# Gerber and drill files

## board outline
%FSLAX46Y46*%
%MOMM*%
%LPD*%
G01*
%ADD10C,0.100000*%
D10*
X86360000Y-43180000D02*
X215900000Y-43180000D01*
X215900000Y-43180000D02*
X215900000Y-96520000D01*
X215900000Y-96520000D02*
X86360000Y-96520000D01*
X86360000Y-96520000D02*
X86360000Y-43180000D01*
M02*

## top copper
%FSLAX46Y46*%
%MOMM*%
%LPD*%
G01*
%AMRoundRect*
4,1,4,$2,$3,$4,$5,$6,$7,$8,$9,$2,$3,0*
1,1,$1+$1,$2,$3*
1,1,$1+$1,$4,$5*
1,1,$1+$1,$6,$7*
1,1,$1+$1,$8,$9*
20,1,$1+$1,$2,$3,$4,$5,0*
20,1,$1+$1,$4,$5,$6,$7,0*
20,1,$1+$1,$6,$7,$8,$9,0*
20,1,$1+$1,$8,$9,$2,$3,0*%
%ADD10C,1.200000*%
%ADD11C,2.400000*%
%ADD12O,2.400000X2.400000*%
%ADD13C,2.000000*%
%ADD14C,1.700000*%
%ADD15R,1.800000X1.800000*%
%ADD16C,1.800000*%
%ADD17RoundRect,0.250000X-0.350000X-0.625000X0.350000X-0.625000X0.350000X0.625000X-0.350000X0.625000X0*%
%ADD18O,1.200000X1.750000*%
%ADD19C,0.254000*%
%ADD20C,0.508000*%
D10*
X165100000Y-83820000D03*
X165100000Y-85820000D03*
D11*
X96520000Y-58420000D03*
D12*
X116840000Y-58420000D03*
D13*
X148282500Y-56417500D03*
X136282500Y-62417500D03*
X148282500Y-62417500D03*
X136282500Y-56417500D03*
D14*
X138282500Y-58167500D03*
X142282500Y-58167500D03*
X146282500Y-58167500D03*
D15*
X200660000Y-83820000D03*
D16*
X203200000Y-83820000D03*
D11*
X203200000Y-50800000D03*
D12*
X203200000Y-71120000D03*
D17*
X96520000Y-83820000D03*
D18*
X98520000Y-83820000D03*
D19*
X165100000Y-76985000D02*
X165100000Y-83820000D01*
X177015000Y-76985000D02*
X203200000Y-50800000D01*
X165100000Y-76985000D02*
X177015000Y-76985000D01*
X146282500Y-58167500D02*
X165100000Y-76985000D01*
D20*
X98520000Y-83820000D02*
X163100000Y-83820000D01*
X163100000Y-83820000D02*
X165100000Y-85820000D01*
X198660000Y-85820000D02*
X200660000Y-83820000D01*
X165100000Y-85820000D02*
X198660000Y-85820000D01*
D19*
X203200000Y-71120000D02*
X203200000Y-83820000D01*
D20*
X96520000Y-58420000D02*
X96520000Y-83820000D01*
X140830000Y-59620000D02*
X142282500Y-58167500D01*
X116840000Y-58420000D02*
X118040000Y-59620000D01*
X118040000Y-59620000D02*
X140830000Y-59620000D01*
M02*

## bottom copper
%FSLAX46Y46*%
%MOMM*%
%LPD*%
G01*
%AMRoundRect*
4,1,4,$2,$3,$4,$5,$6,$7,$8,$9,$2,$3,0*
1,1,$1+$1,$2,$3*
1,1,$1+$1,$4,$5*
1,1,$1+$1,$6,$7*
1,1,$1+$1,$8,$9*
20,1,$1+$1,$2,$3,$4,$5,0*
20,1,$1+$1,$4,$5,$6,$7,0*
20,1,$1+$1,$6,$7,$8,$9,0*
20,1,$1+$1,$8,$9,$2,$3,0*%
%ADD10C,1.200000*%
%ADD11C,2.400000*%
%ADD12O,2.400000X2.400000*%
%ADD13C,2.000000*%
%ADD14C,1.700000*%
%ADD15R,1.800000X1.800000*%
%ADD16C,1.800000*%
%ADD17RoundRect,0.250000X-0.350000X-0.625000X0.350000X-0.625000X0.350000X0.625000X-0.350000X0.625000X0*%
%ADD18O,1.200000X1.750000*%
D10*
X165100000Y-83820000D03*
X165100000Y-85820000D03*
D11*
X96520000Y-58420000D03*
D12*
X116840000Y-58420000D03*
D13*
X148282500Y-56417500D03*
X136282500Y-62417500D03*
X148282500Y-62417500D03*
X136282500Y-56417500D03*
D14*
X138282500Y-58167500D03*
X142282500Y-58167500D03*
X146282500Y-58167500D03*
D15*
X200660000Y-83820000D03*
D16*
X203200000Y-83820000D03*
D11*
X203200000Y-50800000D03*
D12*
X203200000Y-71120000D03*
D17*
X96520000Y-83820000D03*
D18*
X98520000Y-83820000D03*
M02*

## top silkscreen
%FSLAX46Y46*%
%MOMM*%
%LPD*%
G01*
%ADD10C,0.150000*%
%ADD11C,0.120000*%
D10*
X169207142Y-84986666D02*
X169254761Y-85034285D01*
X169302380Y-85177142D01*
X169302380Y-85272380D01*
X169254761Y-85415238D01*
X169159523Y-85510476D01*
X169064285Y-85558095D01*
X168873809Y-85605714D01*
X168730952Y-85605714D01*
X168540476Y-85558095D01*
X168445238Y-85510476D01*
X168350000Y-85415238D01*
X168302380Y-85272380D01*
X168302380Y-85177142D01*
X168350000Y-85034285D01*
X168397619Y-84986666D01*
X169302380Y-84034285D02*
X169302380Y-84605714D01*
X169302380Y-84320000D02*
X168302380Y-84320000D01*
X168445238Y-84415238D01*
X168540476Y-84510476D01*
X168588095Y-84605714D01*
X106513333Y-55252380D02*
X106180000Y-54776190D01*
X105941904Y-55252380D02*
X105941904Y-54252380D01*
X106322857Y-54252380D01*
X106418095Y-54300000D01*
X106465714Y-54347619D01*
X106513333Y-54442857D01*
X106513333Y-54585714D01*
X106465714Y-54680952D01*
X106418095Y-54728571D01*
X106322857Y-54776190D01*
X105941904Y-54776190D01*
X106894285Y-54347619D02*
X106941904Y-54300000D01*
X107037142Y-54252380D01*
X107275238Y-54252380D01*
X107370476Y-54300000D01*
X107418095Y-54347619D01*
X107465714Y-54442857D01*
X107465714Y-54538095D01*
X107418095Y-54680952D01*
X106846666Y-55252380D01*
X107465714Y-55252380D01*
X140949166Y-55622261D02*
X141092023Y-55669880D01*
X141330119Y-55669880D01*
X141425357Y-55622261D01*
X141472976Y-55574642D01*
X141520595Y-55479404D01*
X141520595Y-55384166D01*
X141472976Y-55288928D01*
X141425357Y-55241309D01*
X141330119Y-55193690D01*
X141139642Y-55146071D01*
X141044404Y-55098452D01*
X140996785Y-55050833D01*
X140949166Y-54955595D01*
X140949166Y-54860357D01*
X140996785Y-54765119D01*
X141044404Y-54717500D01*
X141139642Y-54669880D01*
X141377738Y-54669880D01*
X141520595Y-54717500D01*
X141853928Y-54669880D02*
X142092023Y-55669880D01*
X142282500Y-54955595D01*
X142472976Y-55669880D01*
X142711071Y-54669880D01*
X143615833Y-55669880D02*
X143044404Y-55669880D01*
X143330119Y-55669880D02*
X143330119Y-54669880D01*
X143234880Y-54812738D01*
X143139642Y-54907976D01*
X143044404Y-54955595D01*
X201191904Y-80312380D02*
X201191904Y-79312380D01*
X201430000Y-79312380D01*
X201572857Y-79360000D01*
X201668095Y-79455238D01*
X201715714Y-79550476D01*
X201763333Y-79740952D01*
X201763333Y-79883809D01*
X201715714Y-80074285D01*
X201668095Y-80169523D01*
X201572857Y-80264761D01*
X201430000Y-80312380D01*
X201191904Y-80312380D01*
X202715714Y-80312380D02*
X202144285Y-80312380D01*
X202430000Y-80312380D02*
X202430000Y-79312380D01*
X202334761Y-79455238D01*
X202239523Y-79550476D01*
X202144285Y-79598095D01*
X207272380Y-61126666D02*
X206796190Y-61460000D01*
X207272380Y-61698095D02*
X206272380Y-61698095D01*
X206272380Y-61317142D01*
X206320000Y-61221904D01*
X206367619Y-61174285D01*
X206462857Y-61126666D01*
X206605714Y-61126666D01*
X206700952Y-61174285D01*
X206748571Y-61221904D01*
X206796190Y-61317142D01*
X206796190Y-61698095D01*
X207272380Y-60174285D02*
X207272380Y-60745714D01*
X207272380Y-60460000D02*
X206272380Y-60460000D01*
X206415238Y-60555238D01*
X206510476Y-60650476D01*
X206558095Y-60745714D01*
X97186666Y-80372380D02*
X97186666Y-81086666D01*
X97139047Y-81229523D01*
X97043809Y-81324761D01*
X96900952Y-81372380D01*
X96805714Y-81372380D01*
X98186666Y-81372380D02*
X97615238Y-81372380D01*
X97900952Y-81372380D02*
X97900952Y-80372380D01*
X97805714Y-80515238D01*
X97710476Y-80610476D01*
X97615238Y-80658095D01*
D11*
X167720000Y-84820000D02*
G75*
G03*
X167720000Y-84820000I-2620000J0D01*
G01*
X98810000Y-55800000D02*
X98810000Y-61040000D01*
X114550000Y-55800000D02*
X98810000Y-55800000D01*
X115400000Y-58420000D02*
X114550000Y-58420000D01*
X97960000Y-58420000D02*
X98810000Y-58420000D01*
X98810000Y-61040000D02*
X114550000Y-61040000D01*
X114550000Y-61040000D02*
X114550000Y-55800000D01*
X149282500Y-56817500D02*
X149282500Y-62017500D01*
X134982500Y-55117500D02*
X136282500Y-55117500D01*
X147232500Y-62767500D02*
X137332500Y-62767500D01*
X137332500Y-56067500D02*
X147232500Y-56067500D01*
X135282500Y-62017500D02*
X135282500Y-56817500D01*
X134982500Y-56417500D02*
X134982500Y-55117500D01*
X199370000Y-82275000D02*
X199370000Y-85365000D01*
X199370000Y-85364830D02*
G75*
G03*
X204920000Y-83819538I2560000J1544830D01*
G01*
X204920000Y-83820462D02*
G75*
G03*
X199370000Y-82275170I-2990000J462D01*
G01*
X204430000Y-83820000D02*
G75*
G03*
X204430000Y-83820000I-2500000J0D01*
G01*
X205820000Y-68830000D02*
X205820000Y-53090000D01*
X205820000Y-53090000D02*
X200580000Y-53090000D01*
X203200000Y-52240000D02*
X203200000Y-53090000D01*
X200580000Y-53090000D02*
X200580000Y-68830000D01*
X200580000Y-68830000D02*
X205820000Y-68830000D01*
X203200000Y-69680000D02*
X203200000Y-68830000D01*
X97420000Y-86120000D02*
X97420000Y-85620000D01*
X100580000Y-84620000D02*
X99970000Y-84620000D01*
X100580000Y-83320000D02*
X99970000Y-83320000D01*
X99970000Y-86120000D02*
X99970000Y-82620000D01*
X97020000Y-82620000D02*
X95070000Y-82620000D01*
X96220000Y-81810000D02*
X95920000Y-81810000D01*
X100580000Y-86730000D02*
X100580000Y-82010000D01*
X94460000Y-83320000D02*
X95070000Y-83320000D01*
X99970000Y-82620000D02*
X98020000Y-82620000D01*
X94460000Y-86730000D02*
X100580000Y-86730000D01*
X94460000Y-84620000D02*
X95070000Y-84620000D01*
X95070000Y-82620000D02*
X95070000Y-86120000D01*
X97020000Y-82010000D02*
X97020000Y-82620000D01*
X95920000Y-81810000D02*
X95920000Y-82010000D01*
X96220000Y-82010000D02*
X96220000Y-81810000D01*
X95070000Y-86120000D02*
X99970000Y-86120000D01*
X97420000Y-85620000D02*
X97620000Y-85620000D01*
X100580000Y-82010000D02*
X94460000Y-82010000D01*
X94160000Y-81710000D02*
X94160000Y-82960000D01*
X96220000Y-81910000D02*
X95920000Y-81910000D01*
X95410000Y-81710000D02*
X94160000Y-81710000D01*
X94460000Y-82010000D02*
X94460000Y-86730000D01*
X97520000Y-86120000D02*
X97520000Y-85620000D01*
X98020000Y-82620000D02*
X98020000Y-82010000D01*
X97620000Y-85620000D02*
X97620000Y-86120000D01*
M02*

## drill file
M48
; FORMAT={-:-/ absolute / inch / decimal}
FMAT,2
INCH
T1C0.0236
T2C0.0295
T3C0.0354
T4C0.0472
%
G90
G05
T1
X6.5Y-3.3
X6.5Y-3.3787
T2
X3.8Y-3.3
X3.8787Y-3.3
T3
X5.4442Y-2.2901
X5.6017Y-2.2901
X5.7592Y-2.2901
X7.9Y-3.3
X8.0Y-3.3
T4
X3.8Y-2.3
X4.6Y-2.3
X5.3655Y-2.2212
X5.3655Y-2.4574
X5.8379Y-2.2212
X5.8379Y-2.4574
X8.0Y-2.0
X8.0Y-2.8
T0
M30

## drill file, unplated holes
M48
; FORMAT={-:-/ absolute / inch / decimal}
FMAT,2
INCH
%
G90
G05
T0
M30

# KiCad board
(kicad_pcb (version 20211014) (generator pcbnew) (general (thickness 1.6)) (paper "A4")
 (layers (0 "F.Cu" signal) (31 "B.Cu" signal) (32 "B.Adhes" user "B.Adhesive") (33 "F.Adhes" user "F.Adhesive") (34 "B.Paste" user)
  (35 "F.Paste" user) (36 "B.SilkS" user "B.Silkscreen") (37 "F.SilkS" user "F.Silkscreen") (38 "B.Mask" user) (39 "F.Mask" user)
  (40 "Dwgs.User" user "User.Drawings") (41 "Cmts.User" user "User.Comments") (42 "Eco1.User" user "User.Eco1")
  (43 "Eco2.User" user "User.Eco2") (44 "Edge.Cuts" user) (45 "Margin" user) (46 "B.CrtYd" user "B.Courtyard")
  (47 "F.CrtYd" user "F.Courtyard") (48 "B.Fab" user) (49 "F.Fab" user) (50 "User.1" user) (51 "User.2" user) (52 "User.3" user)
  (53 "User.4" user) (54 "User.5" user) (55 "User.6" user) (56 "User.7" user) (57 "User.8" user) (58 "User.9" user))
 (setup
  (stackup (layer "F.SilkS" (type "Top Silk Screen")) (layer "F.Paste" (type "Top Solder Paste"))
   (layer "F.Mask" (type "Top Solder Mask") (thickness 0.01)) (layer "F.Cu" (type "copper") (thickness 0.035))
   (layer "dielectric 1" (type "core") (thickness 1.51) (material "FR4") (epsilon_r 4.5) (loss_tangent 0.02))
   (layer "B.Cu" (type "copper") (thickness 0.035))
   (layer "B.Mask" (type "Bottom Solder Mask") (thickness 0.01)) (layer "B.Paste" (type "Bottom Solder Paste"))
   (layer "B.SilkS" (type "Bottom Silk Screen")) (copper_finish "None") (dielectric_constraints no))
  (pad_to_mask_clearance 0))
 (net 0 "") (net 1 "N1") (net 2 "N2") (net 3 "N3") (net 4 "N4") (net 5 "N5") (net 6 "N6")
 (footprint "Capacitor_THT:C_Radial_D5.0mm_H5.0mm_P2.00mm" (layer "F.Cu") (at 165.1 83.82 -90)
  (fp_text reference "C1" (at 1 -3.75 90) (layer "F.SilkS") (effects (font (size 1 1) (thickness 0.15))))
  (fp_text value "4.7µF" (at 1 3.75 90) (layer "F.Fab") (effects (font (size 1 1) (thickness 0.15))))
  (fp_circle (center 1 0) (end 3.62 0) (layer "F.SilkS") (width 0.12) (fill none))
  (pad "1" thru_hole circle (at 0 0 270) (size 1.2 1.2) (drill 0.6) (layers *.Cu *.Mask) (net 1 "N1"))
  (pad "2" thru_hole circle (at 2 0 270) (size 1.2 1.2) (drill 0.6) (layers *.Cu *.Mask) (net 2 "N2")))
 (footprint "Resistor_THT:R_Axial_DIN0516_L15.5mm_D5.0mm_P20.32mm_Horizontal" (layer "F.Cu") (at 96.52 58.42)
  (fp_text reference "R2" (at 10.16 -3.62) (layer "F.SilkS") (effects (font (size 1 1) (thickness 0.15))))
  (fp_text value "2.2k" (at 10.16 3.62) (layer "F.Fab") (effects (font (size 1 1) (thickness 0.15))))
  (fp_line (start 2.29 -2.62) (end 2.29 2.62) (layer "F.SilkS") (width 0.12))
  (fp_line (start 18.03 -2.62) (end 2.29 -2.62) (layer "F.SilkS") (width 0.12))
  (fp_line (start 18.88 0) (end 18.03 0) (layer "F.SilkS") (width 0.12))
  (fp_line (start 1.44 0) (end 2.29 0) (layer "F.SilkS") (width 0.12))
  (fp_line (start 2.29 2.62) (end 18.03 2.62) (layer "F.SilkS") (width 0.12))
  (fp_line (start 18.03 2.62) (end 18.03 -2.62) (layer "F.SilkS") (width 0.12))
  (pad "1" thru_hole circle (at 0 0) (size 2.4 2.4) (drill 1.2) (layers *.Cu *.Mask) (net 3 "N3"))
  (pad "2" thru_hole oval (at 20.32 0) (size 2.4 2.4) (drill 1.2) (layers *.Cu *.Mask) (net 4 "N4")))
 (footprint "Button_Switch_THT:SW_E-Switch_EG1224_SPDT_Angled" (layer "F.Cu") (at 138.2825 58.1675)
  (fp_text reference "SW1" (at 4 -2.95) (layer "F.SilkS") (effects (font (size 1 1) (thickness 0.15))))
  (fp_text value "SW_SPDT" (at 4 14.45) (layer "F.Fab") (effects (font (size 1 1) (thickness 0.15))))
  (fp_line (start 11 -1.35) (end 11 3.85) (layer "F.SilkS") (width 0.12))
  (fp_line (start -3.3 -3.05) (end -2 -3.05) (layer "F.SilkS") (width 0.12))
  (fp_line (start 8.95 4.6) (end -0.95 4.6) (layer "F.SilkS") (width 0.12))
  (fp_line (start -0.95 -2.1) (end 8.95 -2.1) (layer "F.SilkS") (width 0.12))
  (fp_line (start -3 3.85) (end -3 -1.35) (layer "F.SilkS") (width 0.12))
  (fp_line (start -3.3 -1.75) (end -3.3 -3.05) (layer "F.SilkS") (width 0.12))
  (pad "" thru_hole circle (at 10 -1.75) (size 2 2) (drill 1.2) (layers *.Cu *.Mask))
  (pad "" thru_hole circle (at -2 4.25) (size 2 2) (drill 1.2) (layers *.Cu *.Mask))
  (pad "" thru_hole circle (at 10 4.25) (size 2 2) (drill 1.2) (layers *.Cu *.Mask))
  (pad "" thru_hole circle (at -2 -1.75) (size 2 2) (drill 1.2) (layers *.Cu *.Mask))
  (pad "1" thru_hole circle (at 0 0) (size 1.7 1.7) (drill 0.9) (layers *.Cu *.Mask) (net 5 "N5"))
  (pad "2" thru_hole circle (at 4 0) (size 1.7 1.7) (drill 0.9) (layers *.Cu *.Mask) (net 4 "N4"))
  (pad "3" thru_hole circle (at 8 0) (size 1.7 1.7) (drill 0.9) (layers *.Cu *.Mask) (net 1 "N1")))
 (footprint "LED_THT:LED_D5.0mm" (layer "F.Cu") (at 200.66 83.82)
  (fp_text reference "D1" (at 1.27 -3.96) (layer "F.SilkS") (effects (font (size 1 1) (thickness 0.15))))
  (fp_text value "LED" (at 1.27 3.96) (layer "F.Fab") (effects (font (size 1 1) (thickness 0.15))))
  (fp_line (start -1.29 -1.545) (end -1.29 1.545) (layer "F.SilkS") (width 0.12))
  (fp_arc (start 4.26 -0.000462) (mid 2.072002 2.880433) (end -1.29 1.54483) (layer "F.SilkS") (width 0.12))
  (fp_arc (start -1.29 -1.54483) (mid 2.072002 -2.880433) (end 4.26 0.000462) (layer "F.SilkS") (width 0.12))
  (fp_circle (center 1.27 0) (end 3.77 0) (layer "F.SilkS") (width 0.12) (fill none))
  (pad "1" thru_hole rect (at 0 0) (size 1.8 1.8) (drill 0.9) (layers *.Cu *.Mask) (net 2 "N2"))
  (pad "2" thru_hole circle (at 2.54 0) (size 1.8 1.8) (drill 0.9) (layers *.Cu *.Mask) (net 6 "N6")))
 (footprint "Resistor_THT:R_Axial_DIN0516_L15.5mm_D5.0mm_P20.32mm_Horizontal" (layer "F.Cu") (at 203.2 50.8 -90)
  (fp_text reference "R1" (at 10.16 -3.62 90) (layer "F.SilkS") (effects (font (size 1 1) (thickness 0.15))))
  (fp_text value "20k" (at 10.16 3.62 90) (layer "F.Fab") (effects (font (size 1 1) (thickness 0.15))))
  (fp_line (start 18.03 -2.62) (end 2.29 -2.62) (layer "F.SilkS") (width 0.12))
  (fp_line (start 2.29 -2.62) (end 2.29 2.62) (layer "F.SilkS") (width 0.12))
  (fp_line (start 1.44 0) (end 2.29 0) (layer "F.SilkS") (width 0.12))
  (fp_line (start 2.29 2.62) (end 18.03 2.62) (layer "F.SilkS") (width 0.12))
  (fp_line (start 18.03 2.62) (end 18.03 -2.62) (layer "F.SilkS") (width 0.12))
  (fp_line (start 18.88 0) (end 18.03 0) (layer "F.SilkS") (width 0.12))
  (pad "1" thru_hole circle (at 0 0 270) (size 2.4 2.4) (drill 1.2) (layers *.Cu *.Mask) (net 1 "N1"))
  (pad "2" thru_hole oval (at 20.32 0 270) (size 2.4 2.4) (drill 1.2) (layers *.Cu *.Mask) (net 6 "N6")))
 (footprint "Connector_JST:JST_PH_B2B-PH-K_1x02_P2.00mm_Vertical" (layer "F.Cu") (at 96.52 83.82)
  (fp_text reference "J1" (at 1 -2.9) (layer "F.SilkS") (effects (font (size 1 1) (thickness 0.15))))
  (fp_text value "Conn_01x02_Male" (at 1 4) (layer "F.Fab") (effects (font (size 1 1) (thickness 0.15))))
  (fp_line (start 0.9 2.3) (end 0.9 1.8) (layer "F.SilkS") (width 0.12))
  (fp_line (start 4.06 0.8) (end 3.45 0.8) (layer "F.SilkS") (width 0.12))
  (fp_line (start 4.06 -0.5) (end 3.45 -0.5) (layer "F.SilkS") (width 0.12))
  (fp_line (start 3.45 2.3) (end 3.45 -1.2) (layer "F.SilkS") (width 0.12))
  (fp_line (start 0.5 -1.2) (end -1.45 -1.2) (layer "F.SilkS") (width 0.12))
  (fp_line (start -0.3 -2.01) (end -0.6 -2.01) (layer "F.SilkS") (width 0.12))
  (fp_line (start 4.06 2.91) (end 4.06 -1.81) (layer "F.SilkS") (width 0.12))
  (fp_line (start -2.06 -0.5) (end -1.45 -0.5) (layer "F.SilkS") (width 0.12))
  (fp_line (start 3.45 -1.2) (end 1.5 -1.2) (layer "F.SilkS") (width 0.12))
  (fp_line (start -2.06 2.91) (end 4.06 2.91) (layer "F.SilkS") (width 0.12))
  (fp_line (start -2.06 0.8) (end -1.45 0.8) (layer "F.SilkS") (width 0.12))
  (fp_line (start -1.45 -1.2) (end -1.45 2.3) (layer "F.SilkS") (width 0.12))
  (fp_line (start 0.5 -1.81) (end 0.5 -1.2) (layer "F.SilkS") (width 0.12))
  (fp_line (start -0.6 -2.01) (end -0.6 -1.81) (layer "F.SilkS") (width 0.12))
  (fp_line (start -0.3 -1.81) (end -0.3 -2.01) (layer "F.SilkS") (width 0.12))
  (fp_line (start -1.45 2.3) (end 3.45 2.3) (layer "F.SilkS") (width 0.12))
  (fp_line (start 0.9 1.8) (end 1.1 1.8) (layer "F.SilkS") (width 0.12))
  (fp_line (start 4.06 -1.81) (end -2.06 -1.81) (layer "F.SilkS") (width 0.12))
  (fp_line (start -2.36 -2.11) (end -2.36 -0.86) (layer "F.SilkS") (width 0.12))
  (fp_line (start -0.3 -1.91) (end -0.6 -1.91) (layer "F.SilkS") (width 0.12))
  (fp_line (start -1.11 -2.11) (end -2.36 -2.11) (layer "F.SilkS") (width 0.12))
  (fp_line (start -2.06 -1.81) (end -2.06 2.91) (layer "F.SilkS") (width 0.12))
  (fp_line (start 1 2.3) (end 1 1.8) (layer "F.SilkS") (width 0.12))
  (fp_line (start 1.5 -1.2) (end 1.5 -1.81) (layer "F.SilkS") (width 0.12))
  (fp_line (start 1.1 1.8) (end 1.1 2.3) (layer "F.SilkS") (width 0.12))
  (pad "1" thru_hole roundrect (at 0 0) (size 1.2 1.75) (drill 0.75) (layers *.Cu *.Mask) (roundrect_rratio 0.2083333333) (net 3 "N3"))
  (pad "2" thru_hole oval (at 2 0) (size 1.2 1.75) (drill 0.75) (layers *.Cu *.Mask) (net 2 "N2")))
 (gr_rect (start 86.36 43.18) (end 215.9 96.52) (layer "Edge.Cuts") (width 0.1) (fill none))
 (segment (start 165.1 76.985) (end 165.1 83.82) (width 0.254) (layer "F.Cu") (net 1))
 (segment (start 177.015 76.985) (end 203.2 50.8) (width 0.254) (layer "F.Cu") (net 1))
 (segment (start 165.1 76.985) (end 177.015 76.985) (width 0.254) (layer "F.Cu") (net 1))
 (segment (start 146.2825 58.1675) (end 165.1 76.985) (width 0.254) (layer "F.Cu") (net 1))
 (segment (start 98.52 83.82) (end 163.1 83.82) (width 0.508) (layer "F.Cu") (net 2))
 (segment (start 163.1 83.82) (end 165.1 85.82) (width 0.508) (layer "F.Cu") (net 2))
 (segment (start 198.66 85.82) (end 200.66 83.82) (width 0.508) (layer "F.Cu") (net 2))
 (segment (start 165.1 85.82) (end 198.66 85.82) (width 0.508) (layer "F.Cu") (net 2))
 (segment (start 203.2 71.12) (end 203.2 83.82) (width 0.254) (layer "F.Cu") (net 6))
 (segment (start 96.52 58.42) (end 96.52 83.82) (width 0.508) (layer "F.Cu") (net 3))
 (segment (start 140.83 59.62) (end 142.2825 58.1675) (width 0.508) (layer "F.Cu") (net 4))
 (segment (start 116.84 58.42) (end 118.04 59.62) (width 0.508) (layer "F.Cu") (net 4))
 (segment (start 118.04 59.62) (end 140.83 59.62) (width 0.508) (layer "F.Cu") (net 4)))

